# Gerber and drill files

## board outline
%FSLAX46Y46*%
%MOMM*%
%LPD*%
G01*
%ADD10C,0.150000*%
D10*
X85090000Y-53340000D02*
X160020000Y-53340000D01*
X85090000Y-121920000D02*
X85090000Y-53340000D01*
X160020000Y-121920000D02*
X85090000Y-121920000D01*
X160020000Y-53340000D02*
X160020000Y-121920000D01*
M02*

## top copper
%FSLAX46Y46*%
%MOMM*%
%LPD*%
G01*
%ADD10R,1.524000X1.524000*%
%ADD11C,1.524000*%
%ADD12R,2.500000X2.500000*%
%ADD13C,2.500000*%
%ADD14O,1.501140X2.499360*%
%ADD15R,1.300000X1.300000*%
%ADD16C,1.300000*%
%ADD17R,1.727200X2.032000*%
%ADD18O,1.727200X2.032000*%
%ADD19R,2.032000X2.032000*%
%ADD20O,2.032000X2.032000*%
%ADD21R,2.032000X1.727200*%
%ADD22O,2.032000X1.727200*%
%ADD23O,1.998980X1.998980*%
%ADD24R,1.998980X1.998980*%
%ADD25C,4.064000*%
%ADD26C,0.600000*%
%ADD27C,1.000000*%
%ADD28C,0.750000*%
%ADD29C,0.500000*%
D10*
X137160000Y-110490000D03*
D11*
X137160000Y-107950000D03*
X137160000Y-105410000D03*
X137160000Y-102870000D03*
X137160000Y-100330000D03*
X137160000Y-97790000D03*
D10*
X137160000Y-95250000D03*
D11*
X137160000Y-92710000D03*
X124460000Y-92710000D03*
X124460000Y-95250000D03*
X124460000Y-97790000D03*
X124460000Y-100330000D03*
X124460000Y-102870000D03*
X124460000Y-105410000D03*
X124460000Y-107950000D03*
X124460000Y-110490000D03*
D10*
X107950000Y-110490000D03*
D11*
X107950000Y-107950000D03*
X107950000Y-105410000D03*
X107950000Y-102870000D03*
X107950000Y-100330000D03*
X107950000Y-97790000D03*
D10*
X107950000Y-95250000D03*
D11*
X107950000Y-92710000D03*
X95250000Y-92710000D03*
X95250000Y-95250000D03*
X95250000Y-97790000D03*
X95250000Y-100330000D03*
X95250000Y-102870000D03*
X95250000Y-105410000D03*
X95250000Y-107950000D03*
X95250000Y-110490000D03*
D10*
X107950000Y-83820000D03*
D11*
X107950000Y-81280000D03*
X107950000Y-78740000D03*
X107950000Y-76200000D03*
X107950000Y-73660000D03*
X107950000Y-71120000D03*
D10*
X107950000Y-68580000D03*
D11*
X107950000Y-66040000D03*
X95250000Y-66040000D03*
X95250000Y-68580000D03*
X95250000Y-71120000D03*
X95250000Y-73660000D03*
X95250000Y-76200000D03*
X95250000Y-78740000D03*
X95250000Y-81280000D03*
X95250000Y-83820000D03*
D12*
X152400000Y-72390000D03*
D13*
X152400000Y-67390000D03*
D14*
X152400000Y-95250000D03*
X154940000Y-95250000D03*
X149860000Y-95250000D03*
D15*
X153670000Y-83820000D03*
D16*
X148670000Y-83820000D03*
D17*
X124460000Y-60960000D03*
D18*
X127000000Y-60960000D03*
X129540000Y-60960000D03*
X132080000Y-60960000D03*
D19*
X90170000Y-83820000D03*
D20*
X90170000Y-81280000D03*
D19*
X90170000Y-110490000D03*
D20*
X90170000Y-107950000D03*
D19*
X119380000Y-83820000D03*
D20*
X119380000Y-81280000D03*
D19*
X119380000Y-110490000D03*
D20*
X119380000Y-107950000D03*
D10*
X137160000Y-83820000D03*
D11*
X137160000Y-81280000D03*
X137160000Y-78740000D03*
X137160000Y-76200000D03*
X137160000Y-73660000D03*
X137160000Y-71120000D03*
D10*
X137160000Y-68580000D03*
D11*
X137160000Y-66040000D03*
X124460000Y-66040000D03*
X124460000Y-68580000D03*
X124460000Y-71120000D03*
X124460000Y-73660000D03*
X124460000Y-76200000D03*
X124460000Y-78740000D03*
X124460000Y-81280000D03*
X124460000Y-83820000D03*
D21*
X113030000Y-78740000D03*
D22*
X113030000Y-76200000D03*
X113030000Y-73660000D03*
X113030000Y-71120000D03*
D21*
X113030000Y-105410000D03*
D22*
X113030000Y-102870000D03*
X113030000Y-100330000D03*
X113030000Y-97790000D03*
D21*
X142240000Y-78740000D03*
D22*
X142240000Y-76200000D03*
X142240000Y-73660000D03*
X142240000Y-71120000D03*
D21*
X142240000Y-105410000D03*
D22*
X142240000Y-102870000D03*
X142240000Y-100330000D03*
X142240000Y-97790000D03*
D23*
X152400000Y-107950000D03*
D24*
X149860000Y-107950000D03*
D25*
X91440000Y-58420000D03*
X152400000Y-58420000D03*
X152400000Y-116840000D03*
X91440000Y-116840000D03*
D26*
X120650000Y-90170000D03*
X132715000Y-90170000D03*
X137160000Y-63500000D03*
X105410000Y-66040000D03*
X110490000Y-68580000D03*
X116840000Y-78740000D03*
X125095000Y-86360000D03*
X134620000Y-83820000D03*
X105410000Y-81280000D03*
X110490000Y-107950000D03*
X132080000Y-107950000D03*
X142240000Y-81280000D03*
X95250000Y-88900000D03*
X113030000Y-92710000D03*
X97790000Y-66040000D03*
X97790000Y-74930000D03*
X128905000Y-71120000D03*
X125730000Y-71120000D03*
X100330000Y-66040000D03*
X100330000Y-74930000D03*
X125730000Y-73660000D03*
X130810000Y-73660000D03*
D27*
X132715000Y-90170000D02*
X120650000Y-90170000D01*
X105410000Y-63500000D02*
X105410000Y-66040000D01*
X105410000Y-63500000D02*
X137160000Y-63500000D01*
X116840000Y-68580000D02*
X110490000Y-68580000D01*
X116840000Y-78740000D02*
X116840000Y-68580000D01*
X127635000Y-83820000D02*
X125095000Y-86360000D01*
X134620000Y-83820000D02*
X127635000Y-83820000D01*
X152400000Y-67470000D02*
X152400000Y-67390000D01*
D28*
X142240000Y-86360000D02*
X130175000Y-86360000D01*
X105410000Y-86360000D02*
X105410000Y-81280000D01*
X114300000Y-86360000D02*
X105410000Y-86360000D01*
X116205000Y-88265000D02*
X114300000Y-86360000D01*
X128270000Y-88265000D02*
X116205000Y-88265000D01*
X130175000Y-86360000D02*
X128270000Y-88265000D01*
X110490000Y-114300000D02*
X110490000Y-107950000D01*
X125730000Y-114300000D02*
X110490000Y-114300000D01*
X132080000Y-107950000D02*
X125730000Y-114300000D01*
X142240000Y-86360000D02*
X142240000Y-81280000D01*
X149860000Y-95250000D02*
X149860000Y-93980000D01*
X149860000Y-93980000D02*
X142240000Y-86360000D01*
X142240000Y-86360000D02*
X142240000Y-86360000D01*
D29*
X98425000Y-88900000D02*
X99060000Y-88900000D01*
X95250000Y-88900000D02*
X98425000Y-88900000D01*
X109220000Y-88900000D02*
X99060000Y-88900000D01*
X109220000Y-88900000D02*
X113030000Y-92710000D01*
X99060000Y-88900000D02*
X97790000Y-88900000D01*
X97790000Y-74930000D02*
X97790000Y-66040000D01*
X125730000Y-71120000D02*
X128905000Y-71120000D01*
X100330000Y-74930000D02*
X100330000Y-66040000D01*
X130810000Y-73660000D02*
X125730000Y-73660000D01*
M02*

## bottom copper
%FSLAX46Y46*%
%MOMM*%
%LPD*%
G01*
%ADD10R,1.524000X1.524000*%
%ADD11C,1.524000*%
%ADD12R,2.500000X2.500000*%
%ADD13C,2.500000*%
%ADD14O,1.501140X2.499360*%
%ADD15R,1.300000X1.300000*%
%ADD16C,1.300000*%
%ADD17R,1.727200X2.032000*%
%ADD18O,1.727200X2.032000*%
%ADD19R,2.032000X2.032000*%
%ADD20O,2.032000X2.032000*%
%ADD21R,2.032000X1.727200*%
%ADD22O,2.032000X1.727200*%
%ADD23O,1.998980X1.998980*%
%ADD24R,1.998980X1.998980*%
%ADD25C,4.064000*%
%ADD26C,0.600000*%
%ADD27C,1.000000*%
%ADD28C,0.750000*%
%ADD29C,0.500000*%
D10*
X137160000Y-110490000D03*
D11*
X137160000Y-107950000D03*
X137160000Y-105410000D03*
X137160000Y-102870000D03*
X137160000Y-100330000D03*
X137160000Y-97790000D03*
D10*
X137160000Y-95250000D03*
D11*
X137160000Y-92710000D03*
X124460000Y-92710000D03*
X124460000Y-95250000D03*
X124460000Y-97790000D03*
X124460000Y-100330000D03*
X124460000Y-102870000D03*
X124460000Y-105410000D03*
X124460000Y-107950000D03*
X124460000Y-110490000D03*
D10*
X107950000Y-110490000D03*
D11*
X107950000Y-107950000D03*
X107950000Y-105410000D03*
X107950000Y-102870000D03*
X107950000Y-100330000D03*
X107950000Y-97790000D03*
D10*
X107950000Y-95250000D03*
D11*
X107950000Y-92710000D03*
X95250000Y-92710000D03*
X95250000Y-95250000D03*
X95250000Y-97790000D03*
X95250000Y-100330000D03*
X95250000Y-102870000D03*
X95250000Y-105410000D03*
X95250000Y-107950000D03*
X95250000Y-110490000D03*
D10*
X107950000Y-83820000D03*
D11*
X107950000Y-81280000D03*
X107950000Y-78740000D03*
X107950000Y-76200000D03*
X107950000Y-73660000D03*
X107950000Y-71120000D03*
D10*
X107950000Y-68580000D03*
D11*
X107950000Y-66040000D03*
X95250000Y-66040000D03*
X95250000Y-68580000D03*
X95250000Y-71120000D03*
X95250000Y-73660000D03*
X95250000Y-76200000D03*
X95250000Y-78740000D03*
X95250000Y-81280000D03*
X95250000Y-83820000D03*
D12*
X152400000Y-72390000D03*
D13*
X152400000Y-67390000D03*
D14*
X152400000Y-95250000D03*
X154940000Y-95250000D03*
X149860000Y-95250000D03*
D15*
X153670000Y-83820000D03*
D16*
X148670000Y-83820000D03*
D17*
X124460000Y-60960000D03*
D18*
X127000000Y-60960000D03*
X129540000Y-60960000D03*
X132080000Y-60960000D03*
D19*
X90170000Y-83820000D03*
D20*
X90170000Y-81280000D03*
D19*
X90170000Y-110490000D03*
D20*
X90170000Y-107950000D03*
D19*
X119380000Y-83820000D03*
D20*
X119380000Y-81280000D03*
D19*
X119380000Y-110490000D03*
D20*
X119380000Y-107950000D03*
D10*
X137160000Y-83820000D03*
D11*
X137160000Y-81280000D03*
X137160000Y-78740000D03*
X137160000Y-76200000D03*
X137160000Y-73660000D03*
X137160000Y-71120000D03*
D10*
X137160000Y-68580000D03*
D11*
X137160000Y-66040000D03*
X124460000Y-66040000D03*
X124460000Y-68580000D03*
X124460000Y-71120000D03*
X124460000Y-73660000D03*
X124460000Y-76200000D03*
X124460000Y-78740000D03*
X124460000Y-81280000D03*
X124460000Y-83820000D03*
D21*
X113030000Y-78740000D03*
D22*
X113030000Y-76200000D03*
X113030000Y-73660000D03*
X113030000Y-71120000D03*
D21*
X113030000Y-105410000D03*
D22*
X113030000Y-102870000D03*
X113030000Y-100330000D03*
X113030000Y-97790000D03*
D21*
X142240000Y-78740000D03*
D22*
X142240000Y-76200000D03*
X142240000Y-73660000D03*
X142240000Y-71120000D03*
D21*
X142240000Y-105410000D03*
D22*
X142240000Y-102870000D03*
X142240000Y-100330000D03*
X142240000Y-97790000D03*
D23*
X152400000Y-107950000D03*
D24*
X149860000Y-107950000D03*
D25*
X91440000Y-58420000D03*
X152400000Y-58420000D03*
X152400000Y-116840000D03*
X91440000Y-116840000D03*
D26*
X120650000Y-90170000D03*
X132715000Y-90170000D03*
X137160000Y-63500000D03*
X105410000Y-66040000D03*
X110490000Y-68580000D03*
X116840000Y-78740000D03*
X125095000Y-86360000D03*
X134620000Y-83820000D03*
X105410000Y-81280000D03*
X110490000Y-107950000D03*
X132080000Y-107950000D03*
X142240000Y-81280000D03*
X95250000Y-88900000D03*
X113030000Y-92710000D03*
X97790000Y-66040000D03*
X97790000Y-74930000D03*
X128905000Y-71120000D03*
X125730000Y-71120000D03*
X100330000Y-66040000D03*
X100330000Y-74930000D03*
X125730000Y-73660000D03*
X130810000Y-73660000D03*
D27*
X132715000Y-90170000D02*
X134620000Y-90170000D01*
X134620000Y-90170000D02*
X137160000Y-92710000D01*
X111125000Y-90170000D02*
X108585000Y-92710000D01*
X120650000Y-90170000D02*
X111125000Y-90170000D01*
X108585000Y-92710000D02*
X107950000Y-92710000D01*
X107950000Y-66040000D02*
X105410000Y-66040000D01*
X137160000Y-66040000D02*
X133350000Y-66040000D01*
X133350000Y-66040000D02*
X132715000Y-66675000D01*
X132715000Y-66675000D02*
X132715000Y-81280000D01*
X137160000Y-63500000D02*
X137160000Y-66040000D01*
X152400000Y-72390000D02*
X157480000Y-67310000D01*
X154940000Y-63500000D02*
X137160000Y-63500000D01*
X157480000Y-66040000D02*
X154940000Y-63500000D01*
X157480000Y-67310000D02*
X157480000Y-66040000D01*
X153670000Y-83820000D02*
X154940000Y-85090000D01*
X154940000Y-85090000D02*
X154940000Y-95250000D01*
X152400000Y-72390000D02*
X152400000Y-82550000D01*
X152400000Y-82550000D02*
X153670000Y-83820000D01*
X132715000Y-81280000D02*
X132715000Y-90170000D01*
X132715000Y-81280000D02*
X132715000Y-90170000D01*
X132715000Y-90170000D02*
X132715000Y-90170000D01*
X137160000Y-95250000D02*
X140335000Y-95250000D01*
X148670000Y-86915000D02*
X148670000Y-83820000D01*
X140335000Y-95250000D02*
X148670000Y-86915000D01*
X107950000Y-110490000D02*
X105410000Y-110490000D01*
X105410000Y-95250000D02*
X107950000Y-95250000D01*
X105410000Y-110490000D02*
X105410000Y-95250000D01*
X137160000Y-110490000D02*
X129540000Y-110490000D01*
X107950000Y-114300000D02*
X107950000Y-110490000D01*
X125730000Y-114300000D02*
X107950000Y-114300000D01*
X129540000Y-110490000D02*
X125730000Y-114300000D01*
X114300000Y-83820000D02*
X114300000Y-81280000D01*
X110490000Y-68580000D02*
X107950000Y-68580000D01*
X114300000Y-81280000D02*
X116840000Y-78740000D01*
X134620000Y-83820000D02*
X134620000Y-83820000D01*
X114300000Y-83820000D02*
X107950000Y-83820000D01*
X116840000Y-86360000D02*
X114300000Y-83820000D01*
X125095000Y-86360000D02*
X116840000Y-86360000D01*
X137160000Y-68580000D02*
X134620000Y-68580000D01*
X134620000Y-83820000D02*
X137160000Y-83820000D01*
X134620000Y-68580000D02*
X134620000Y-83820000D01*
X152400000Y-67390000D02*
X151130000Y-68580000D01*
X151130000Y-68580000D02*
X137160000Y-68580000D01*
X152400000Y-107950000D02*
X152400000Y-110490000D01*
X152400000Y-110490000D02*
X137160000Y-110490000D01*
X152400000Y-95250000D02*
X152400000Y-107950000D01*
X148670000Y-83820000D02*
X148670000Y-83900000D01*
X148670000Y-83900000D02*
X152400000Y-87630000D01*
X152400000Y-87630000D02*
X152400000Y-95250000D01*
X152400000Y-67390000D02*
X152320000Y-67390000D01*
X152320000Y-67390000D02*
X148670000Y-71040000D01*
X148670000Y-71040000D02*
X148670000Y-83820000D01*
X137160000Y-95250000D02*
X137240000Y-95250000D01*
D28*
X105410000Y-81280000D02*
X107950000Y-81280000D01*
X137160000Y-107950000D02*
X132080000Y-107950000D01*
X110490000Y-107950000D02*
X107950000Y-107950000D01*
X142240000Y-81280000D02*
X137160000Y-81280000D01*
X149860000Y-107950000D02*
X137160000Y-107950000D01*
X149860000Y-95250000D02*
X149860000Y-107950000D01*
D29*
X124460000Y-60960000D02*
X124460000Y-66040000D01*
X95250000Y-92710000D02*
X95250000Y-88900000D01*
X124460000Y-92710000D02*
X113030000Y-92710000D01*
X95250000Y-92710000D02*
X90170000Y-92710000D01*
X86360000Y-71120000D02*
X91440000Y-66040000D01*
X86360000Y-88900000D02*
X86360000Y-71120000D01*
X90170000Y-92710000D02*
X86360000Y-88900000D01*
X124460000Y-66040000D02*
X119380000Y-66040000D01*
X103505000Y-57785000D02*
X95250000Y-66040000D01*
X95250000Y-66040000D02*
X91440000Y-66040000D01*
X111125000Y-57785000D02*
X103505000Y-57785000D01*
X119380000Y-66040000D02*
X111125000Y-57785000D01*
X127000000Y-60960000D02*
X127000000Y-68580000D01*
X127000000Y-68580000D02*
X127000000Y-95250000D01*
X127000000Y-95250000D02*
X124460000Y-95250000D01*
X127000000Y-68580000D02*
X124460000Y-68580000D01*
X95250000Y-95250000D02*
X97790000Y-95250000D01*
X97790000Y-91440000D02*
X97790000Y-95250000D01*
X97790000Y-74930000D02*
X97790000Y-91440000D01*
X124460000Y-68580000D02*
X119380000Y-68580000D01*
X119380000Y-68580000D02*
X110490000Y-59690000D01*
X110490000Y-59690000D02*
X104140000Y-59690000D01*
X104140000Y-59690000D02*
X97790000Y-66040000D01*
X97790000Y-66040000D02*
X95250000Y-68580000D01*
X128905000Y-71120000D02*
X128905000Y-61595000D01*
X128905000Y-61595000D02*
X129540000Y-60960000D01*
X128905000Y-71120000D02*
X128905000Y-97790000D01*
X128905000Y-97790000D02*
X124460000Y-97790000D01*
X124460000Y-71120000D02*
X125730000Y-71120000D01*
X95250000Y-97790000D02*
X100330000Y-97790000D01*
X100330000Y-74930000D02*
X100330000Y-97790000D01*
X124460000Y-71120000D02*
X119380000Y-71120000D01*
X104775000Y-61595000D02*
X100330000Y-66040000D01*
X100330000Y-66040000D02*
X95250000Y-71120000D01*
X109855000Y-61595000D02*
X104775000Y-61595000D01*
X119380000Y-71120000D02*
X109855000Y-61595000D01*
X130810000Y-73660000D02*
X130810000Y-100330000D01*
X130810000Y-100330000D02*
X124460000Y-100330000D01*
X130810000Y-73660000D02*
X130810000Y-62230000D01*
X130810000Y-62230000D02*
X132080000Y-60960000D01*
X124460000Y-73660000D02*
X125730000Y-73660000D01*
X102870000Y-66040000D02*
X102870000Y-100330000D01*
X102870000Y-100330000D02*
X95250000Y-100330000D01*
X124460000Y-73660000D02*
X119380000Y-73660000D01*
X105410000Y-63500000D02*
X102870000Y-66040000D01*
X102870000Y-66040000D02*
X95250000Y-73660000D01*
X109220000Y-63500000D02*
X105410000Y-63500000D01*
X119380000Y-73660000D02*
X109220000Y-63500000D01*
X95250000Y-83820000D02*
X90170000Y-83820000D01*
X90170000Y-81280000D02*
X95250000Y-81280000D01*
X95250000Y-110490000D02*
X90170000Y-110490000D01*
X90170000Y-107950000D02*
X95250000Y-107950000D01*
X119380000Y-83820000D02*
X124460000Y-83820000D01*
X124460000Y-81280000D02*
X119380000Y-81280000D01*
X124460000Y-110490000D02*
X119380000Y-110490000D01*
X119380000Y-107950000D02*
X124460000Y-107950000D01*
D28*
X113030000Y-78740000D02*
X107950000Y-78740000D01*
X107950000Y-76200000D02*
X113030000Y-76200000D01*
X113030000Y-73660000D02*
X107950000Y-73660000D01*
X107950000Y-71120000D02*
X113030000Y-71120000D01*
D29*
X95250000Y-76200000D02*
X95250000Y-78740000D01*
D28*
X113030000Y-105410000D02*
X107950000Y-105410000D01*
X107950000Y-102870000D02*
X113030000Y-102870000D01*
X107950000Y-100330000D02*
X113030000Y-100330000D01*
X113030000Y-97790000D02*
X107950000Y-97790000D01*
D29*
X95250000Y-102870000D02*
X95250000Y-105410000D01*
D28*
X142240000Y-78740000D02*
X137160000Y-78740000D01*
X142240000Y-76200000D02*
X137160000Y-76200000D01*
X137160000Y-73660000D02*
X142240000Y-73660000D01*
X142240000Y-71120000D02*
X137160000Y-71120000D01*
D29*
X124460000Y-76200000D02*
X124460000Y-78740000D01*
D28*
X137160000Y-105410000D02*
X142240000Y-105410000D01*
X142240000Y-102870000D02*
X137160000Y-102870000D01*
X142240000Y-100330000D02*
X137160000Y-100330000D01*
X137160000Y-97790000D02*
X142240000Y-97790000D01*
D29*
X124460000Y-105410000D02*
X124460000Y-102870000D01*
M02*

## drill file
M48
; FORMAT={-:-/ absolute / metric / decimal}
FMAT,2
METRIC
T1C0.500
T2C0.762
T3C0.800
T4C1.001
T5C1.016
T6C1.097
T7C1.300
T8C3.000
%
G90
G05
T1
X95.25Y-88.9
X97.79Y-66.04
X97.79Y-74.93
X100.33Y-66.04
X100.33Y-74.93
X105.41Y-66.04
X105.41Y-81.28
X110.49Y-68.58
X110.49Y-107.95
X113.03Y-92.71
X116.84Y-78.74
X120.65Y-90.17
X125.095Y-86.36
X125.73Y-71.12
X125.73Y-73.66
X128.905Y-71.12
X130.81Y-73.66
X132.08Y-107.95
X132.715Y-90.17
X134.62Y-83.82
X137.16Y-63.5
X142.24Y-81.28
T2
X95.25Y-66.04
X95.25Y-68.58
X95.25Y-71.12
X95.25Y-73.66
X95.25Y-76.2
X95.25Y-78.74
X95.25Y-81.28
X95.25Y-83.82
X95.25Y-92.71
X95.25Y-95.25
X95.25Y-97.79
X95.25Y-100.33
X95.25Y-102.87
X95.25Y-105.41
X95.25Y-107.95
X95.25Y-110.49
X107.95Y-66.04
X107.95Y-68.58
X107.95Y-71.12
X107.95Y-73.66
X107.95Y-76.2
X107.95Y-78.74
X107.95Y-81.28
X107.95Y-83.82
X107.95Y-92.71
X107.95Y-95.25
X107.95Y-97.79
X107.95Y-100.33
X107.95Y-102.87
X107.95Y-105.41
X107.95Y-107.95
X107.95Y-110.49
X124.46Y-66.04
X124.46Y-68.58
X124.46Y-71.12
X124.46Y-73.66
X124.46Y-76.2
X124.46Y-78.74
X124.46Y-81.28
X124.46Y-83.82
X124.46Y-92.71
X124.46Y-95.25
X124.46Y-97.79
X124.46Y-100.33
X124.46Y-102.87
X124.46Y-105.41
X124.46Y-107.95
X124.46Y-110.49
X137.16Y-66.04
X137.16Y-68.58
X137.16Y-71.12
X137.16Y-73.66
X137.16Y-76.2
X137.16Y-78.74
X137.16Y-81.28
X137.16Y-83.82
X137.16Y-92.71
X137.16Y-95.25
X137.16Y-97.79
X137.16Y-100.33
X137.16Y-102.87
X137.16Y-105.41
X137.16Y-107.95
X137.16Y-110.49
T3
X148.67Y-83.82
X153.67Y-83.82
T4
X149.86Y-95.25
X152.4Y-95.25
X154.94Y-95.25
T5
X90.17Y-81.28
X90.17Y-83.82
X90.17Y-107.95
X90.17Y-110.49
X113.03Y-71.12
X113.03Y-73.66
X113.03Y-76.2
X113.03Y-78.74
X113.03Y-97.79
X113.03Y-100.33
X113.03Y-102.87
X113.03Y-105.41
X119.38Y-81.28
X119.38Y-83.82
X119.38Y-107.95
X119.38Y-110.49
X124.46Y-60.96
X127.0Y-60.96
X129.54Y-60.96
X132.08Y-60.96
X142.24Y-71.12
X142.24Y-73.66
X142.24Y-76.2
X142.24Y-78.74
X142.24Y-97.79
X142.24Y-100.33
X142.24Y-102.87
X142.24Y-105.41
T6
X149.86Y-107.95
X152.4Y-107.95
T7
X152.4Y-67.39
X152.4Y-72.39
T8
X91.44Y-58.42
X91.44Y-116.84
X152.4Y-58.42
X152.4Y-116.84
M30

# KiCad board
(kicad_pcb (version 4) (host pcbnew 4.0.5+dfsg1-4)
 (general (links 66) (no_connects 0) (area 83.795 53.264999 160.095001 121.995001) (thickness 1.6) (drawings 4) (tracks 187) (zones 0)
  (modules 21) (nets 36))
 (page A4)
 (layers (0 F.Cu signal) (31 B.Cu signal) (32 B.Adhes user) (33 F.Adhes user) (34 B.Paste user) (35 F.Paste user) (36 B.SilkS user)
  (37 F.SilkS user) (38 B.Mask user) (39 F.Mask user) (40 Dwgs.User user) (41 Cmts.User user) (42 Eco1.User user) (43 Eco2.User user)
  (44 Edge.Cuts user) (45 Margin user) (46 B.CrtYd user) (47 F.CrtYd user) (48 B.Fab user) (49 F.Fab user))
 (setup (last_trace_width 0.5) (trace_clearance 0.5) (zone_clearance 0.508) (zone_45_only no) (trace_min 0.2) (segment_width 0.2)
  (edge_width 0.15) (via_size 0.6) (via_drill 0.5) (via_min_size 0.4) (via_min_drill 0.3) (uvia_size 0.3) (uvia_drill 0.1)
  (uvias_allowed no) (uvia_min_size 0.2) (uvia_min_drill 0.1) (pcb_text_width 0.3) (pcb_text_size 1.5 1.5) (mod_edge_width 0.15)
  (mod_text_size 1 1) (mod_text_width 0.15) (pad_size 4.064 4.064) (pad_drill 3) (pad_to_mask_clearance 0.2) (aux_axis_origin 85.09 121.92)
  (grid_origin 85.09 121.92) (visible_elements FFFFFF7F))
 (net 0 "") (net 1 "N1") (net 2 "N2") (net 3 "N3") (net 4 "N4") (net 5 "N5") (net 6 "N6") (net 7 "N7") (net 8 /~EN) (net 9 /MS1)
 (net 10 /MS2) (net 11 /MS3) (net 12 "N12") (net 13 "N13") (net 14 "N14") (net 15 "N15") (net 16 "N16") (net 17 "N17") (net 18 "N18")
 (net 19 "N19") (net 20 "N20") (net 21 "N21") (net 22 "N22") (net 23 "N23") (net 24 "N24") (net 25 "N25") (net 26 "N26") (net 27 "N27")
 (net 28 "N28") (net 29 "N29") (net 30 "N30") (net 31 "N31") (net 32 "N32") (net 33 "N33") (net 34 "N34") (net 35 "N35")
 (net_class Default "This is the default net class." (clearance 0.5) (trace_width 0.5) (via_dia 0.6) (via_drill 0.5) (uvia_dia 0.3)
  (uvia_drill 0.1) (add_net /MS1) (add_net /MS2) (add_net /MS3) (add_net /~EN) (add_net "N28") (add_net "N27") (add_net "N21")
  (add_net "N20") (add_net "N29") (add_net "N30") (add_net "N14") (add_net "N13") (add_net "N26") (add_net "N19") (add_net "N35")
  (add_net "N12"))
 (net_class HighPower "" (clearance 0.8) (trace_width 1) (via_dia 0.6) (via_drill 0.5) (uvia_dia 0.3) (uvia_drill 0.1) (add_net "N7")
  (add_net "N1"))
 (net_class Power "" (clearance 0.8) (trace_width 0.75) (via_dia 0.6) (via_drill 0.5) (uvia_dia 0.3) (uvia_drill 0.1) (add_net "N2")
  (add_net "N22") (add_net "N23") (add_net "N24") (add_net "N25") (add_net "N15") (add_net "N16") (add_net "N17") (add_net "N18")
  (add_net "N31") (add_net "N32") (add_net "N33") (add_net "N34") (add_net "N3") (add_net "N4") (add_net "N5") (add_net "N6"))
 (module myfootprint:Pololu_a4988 (layer F.Cu) (at 130.81 101.6)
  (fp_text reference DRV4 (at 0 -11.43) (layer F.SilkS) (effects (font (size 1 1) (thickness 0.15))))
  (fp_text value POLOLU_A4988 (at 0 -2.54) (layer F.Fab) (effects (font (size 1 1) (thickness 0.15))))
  (pad 1 thru_hole rect (at 6.35 8.89) (size 1.524 1.524) (drill 0.762) (layers *.Cu *.Mask) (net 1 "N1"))
  (pad 2 thru_hole circle (at 6.35 6.35) (size 1.524 1.524) (drill 0.762) (layers *.Cu *.Mask) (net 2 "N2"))
  (pad 3 thru_hole circle (at 6.35 3.81) (size 1.524 1.524) (drill 0.762) (layers *.Cu *.Mask) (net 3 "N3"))
  (pad 4 thru_hole circle (at 6.35 1.27) (size 1.524 1.524) (drill 0.762) (layers *.Cu *.Mask) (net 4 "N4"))
  (pad 5 thru_hole circle (at 6.35 -1.27) (size 1.524 1.524) (drill 0.762) (layers *.Cu *.Mask) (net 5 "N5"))
  (pad 6 thru_hole circle (at 6.35 -3.81) (size 1.524 1.524) (drill 0.762) (layers *.Cu *.Mask) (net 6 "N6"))
  (pad 7 thru_hole rect (at 6.35 -6.35) (size 1.524 1.524) (drill 0.762) (layers *.Cu *.Mask) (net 1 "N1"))
  (pad 8 thru_hole circle (at 6.35 -8.89) (size 1.524 1.524) (drill 0.762) (layers *.Cu *.Mask) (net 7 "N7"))
  (pad 9 thru_hole circle (at -6.35 -8.89) (size 1.524 1.524) (drill 0.762) (layers *.Cu *.Mask) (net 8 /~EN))
  (pad 10 thru_hole circle (at -6.35 -6.35) (size 1.524 1.524) (drill 0.762) (layers *.Cu *.Mask) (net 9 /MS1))
  (pad 11 thru_hole circle (at -6.35 -3.81) (size 1.524 1.524) (drill 0.762) (layers *.Cu *.Mask) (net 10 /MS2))
  (pad 12 thru_hole circle (at -6.35 -1.27) (size 1.524 1.524) (drill 0.762) (layers *.Cu *.Mask) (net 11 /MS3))
  (pad 13 thru_hole circle (at -6.35 1.27) (size 1.524 1.524) (drill 0.762) (layers *.Cu *.Mask) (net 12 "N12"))
  (pad 14 thru_hole circle (at -6.35 3.81) (size 1.524 1.524) (drill 0.762) (layers *.Cu *.Mask) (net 12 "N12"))
  (pad 15 thru_hole circle (at -6.35 6.35) (size 1.524 1.524) (drill 0.762) (layers *.Cu *.Mask) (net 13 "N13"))
  (pad 16 thru_hole circle (at -6.35 8.89) (size 1.524 1.524) (drill 0.762) (layers *.Cu *.Mask) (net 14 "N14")))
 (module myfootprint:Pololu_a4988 (layer F.Cu) (at 101.6 101.6)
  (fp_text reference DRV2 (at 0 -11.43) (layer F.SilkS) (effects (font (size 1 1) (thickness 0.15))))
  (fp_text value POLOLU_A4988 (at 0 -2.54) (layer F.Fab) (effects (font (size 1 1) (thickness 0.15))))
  (pad 1 thru_hole rect (at 6.35 8.89) (size 1.524 1.524) (drill 0.762) (layers *.Cu *.Mask) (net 1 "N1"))
  (pad 2 thru_hole circle (at 6.35 6.35) (size 1.524 1.524) (drill 0.762) (layers *.Cu *.Mask) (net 2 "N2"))
  (pad 3 thru_hole circle (at 6.35 3.81) (size 1.524 1.524) (drill 0.762) (layers *.Cu *.Mask) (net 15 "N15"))
  (pad 4 thru_hole circle (at 6.35 1.27) (size 1.524 1.524) (drill 0.762) (layers *.Cu *.Mask) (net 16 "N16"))
  (pad 5 thru_hole circle (at 6.35 -1.27) (size 1.524 1.524) (drill 0.762) (layers *.Cu *.Mask) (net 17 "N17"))
  (pad 6 thru_hole circle (at 6.35 -3.81) (size 1.524 1.524) (drill 0.762) (layers *.Cu *.Mask) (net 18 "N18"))
  (pad 7 thru_hole rect (at 6.35 -6.35) (size 1.524 1.524) (drill 0.762) (layers *.Cu *.Mask) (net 1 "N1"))
  (pad 8 thru_hole circle (at 6.35 -8.89) (size 1.524 1.524) (drill 0.762) (layers *.Cu *.Mask) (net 7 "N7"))
  (pad 9 thru_hole circle (at -6.35 -8.89) (size 1.524 1.524) (drill 0.762) (layers *.Cu *.Mask) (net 8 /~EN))
  (pad 10 thru_hole circle (at -6.35 -6.35) (size 1.524 1.524) (drill 0.762) (layers *.Cu *.Mask) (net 9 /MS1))
  (pad 11 thru_hole circle (at -6.35 -3.81) (size 1.524 1.524) (drill 0.762) (layers *.Cu *.Mask) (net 10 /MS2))
  (pad 12 thru_hole circle (at -6.35 -1.27) (size 1.524 1.524) (drill 0.762) (layers *.Cu *.Mask) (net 11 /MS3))
  (pad 13 thru_hole circle (at -6.35 1.27) (size 1.524 1.524) (drill 0.762) (layers *.Cu *.Mask) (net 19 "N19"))
  (pad 14 thru_hole circle (at -6.35 3.81) (size 1.524 1.524) (drill 0.762) (layers *.Cu *.Mask) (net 19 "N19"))
  (pad 15 thru_hole circle (at -6.35 6.35) (size 1.524 1.524) (drill 0.762) (layers *.Cu *.Mask) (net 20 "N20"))
  (pad 16 thru_hole circle (at -6.35 8.89) (size 1.524 1.524) (drill 0.762) (layers *.Cu *.Mask) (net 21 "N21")))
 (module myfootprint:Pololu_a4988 (layer F.Cu) (at 101.6 74.93)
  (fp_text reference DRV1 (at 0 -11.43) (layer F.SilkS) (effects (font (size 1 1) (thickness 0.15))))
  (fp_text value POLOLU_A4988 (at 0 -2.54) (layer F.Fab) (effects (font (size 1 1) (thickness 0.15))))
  (pad 1 thru_hole rect (at 6.35 8.89) (size 1.524 1.524) (drill 0.762) (layers *.Cu *.Mask) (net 1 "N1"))
  (pad 2 thru_hole circle (at 6.35 6.35) (size 1.524 1.524) (drill 0.762) (layers *.Cu *.Mask) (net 2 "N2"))
  (pad 3 thru_hole circle (at 6.35 3.81) (size 1.524 1.524) (drill 0.762) (layers *.Cu *.Mask) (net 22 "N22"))
  (pad 4 thru_hole circle (at 6.35 1.27) (size 1.524 1.524) (drill 0.762) (layers *.Cu *.Mask) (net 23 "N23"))
  (pad 5 thru_hole circle (at 6.35 -1.27) (size 1.524 1.524) (drill 0.762) (layers *.Cu *.Mask) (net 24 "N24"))
  (pad 6 thru_hole circle (at 6.35 -3.81) (size 1.524 1.524) (drill 0.762) (layers *.Cu *.Mask) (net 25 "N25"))
  (pad 7 thru_hole rect (at 6.35 -6.35) (size 1.524 1.524) (drill 0.762) (layers *.Cu *.Mask) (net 1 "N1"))
  (pad 8 thru_hole circle (at 6.35 -8.89) (size 1.524 1.524) (drill 0.762) (layers *.Cu *.Mask) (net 7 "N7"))
  (pad 9 thru_hole circle (at -6.35 -8.89) (size 1.524 1.524) (drill 0.762) (layers *.Cu *.Mask) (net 8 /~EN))
  (pad 10 thru_hole circle (at -6.35 -6.35) (size 1.524 1.524) (drill 0.762) (layers *.Cu *.Mask) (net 9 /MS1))
  (pad 11 thru_hole circle (at -6.35 -3.81) (size 1.524 1.524) (drill 0.762) (layers *.Cu *.Mask) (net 10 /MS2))
  (pad 12 thru_hole circle (at -6.35 -1.27) (size 1.524 1.524) (drill 0.762) (layers *.Cu *.Mask) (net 11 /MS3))
  (pad 13 thru_hole circle (at -6.35 1.27) (size 1.524 1.524) (drill 0.762) (layers *.Cu *.Mask) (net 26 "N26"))
  (pad 14 thru_hole circle (at -6.35 3.81) (size 1.524 1.524) (drill 0.762) (layers *.Cu *.Mask) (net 26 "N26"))
  (pad 15 thru_hole circle (at -6.35 6.35) (size 1.524 1.524) (drill 0.762) (layers *.Cu *.Mask) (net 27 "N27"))
  (pad 16 thru_hole circle (at -6.35 8.89) (size 1.524 1.524) (drill 0.762) (layers *.Cu *.Mask) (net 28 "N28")))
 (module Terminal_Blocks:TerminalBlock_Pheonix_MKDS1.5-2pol (layer F.Cu) (at 152.4 72.39 90)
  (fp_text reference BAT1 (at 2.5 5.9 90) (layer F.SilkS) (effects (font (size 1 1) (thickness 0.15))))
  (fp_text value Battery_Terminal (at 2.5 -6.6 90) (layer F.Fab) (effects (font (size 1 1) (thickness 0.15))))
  (pad 1 thru_hole rect (at 0 0 90) (size 2.5 2.5) (drill 1.3) (layers *.Cu *.Mask) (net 7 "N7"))
  (pad 2 thru_hole circle (at 5 0 90) (size 2.5 2.5) (drill 1.3) (layers *.Cu *.Mask) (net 1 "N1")))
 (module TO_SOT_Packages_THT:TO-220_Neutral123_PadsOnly (layer F.Cu) (at 152.4 95.25 180)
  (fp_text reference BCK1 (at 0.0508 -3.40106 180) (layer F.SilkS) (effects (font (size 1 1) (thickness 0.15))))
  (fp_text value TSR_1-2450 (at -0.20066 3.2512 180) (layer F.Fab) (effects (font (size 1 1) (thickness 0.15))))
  (pad 2 thru_hole oval (at 0 0 270) (size 2.49936 1.50114) (drill 1.00076) (layers *.Cu *.Mask) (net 1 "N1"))
  (pad 1 thru_hole oval (at -2.54 0 270) (size 2.49936 1.50114) (drill 1.00076) (layers *.Cu *.Mask) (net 7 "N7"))
  (pad 3 thru_hole oval (at 2.54 0 270) (size 2.49936 1.50114) (drill 1.00076) (layers *.Cu *.Mask) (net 2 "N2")))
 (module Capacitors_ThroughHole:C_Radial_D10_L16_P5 (layer F.Cu) (at 153.67 83.82 180)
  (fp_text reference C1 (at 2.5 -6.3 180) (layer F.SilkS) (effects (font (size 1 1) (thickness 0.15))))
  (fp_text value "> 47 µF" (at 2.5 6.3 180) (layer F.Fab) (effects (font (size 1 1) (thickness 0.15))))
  (pad 1 thru_hole rect (at 0 0 180) (size 1.3 1.3) (drill 0.8) (layers *.Cu *.Mask) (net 7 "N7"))
  (pad 2 thru_hole circle (at 5 0 180) (size 1.3 1.3) (drill 0.8) (layers *.Cu *.Mask) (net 1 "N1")))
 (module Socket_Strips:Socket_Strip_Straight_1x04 (layer F.Cu) (at 124.46 60.96)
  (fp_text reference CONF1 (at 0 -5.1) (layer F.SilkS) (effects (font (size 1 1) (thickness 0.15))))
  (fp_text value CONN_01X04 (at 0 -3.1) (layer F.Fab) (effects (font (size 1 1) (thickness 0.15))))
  (pad 1 thru_hole rect (at 0 0) (size 1.7272 2.032) (drill 1.016) (layers *.Cu *.Mask) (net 8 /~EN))
  (pad 2 thru_hole oval (at 2.54 0) (size 1.7272 2.032) (drill 1.016) (layers *.Cu *.Mask) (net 9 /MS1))
  (pad 3 thru_hole oval (at 5.08 0) (size 1.7272 2.032) (drill 1.016) (layers *.Cu *.Mask) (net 10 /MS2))
  (pad 4 thru_hole oval (at 7.62 0) (size 1.7272 2.032) (drill 1.016) (layers *.Cu *.Mask) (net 11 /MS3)))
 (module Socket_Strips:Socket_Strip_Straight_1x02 (layer F.Cu) (at 90.17 83.82 90)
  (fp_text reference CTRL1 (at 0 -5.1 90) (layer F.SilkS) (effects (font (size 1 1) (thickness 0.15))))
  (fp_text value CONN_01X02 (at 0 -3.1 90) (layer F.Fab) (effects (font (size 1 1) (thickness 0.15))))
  (pad 1 thru_hole rect (at 0 0 90) (size 2.032 2.032) (drill 1.016) (layers *.Cu *.Mask) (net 28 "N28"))
  (pad 2 thru_hole oval (at 2.54 0 90) (size 2.032 2.032) (drill 1.016) (layers *.Cu *.Mask) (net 27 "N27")))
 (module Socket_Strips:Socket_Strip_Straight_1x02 (layer F.Cu) (at 90.17 110.49 90)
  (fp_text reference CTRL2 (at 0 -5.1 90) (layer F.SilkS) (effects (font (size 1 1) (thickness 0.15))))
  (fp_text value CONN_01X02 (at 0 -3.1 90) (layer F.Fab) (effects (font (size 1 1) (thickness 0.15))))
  (pad 1 thru_hole rect (at 0 0 90) (size 2.032 2.032) (drill 1.016) (layers *.Cu *.Mask) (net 21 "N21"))
  (pad 2 thru_hole oval (at 2.54 0 90) (size 2.032 2.032) (drill 1.016) (layers *.Cu *.Mask) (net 20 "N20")))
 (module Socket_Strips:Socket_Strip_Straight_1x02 (layer F.Cu) (at 119.38 83.82 90)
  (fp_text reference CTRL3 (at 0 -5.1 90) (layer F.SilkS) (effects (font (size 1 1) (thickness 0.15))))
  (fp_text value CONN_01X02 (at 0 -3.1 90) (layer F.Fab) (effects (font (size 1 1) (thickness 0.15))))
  (pad 1 thru_hole rect (at 0 0 90) (size 2.032 2.032) (drill 1.016) (layers *.Cu *.Mask) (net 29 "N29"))
  (pad 2 thru_hole oval (at 2.54 0 90) (size 2.032 2.032) (drill 1.016) (layers *.Cu *.Mask) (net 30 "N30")))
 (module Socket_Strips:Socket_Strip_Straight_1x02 (layer F.Cu) (at 119.38 110.49 90)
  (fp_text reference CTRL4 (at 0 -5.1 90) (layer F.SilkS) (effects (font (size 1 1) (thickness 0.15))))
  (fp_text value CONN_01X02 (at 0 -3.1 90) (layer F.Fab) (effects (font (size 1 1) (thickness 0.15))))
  (pad 1 thru_hole rect (at 0 0 90) (size 2.032 2.032) (drill 1.016) (layers *.Cu *.Mask) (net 14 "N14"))
  (pad 2 thru_hole oval (at 2.54 0 90) (size 2.032 2.032) (drill 1.016) (layers *.Cu *.Mask) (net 13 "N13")))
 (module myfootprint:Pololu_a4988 (layer F.Cu) (at 130.81 74.93)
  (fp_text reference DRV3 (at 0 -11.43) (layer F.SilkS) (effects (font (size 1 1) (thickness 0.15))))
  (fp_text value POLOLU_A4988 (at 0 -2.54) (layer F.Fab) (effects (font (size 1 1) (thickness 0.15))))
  (pad 1 thru_hole rect (at 6.35 8.89) (size 1.524 1.524) (drill 0.762) (layers *.Cu *.Mask) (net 1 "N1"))
  (pad 2 thru_hole circle (at 6.35 6.35) (size 1.524 1.524) (drill 0.762) (layers *.Cu *.Mask) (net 2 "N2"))
  (pad 3 thru_hole circle (at 6.35 3.81) (size 1.524 1.524) (drill 0.762) (layers *.Cu *.Mask) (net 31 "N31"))
  (pad 4 thru_hole circle (at 6.35 1.27) (size 1.524 1.524) (drill 0.762) (layers *.Cu *.Mask) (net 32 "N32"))
  (pad 5 thru_hole circle (at 6.35 -1.27) (size 1.524 1.524) (drill 0.762) (layers *.Cu *.Mask) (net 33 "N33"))
  (pad 6 thru_hole circle (at 6.35 -3.81) (size 1.524 1.524) (drill 0.762) (layers *.Cu *.Mask) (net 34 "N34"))
  (pad 7 thru_hole rect (at 6.35 -6.35) (size 1.524 1.524) (drill 0.762) (layers *.Cu *.Mask) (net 1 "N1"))
  (pad 8 thru_hole circle (at 6.35 -8.89) (size 1.524 1.524) (drill 0.762) (layers *.Cu *.Mask) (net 7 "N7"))
  (pad 9 thru_hole circle (at -6.35 -8.89) (size 1.524 1.524) (drill 0.762) (layers *.Cu *.Mask) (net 8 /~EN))
  (pad 10 thru_hole circle (at -6.35 -6.35) (size 1.524 1.524) (drill 0.762) (layers *.Cu *.Mask) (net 9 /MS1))
  (pad 11 thru_hole circle (at -6.35 -3.81) (size 1.524 1.524) (drill 0.762) (layers *.Cu *.Mask) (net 10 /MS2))
  (pad 12 thru_hole circle (at -6.35 -1.27) (size 1.524 1.524) (drill 0.762) (layers *.Cu *.Mask) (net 11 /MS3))
  (pad 13 thru_hole circle (at -6.35 1.27) (size 1.524 1.524) (drill 0.762) (layers *.Cu *.Mask) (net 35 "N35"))
  (pad 14 thru_hole circle (at -6.35 3.81) (size 1.524 1.524) (drill 0.762) (layers *.Cu *.Mask) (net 35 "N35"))
  (pad 15 thru_hole circle (at -6.35 6.35) (size 1.524 1.524) (drill 0.762) (layers *.Cu *.Mask) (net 30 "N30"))
  (pad 16 thru_hole circle (at -6.35 8.89) (size 1.524 1.524) (drill 0.762) (layers *.Cu *.Mask) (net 29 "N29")))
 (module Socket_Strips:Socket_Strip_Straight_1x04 (layer F.Cu) (at 113.03 78.74 90)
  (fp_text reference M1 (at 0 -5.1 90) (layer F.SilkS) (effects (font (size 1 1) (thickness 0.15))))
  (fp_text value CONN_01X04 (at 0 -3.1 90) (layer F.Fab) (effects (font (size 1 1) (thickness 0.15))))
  (pad 1 thru_hole rect (at 0 0 90) (size 1.7272 2.032) (drill 1.016) (layers *.Cu *.Mask) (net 22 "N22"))
  (pad 2 thru_hole oval (at 2.54 0 90) (size 1.7272 2.032) (drill 1.016) (layers *.Cu *.Mask) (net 23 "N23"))
  (pad 3 thru_hole oval (at 5.08 0 90) (size 1.7272 2.032) (drill 1.016) (layers *.Cu *.Mask) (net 24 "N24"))
  (pad 4 thru_hole oval (at 7.62 0 90) (size 1.7272 2.032) (drill 1.016) (layers *.Cu *.Mask) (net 25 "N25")))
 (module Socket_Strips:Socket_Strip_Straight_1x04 (layer F.Cu) (at 113.03 105.41 90)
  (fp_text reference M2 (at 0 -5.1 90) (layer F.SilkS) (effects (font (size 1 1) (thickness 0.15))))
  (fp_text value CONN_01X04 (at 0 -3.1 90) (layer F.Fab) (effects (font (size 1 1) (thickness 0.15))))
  (pad 1 thru_hole rect (at 0 0 90) (size 1.7272 2.032) (drill 1.016) (layers *.Cu *.Mask) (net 15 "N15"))
  (pad 2 thru_hole oval (at 2.54 0 90) (size 1.7272 2.032) (drill 1.016) (layers *.Cu *.Mask) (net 16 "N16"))
  (pad 3 thru_hole oval (at 5.08 0 90) (size 1.7272 2.032) (drill 1.016) (layers *.Cu *.Mask) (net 17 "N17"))
  (pad 4 thru_hole oval (at 7.62 0 90) (size 1.7272 2.032) (drill 1.016) (layers *.Cu *.Mask) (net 18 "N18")))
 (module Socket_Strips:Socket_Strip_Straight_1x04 (layer F.Cu) (at 142.24 78.74 90)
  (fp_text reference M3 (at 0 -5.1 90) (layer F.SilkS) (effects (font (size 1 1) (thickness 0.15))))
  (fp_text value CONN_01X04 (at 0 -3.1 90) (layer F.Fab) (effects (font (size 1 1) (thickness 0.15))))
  (pad 1 thru_hole rect (at 0 0 90) (size 1.7272 2.032) (drill 1.016) (layers *.Cu *.Mask) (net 31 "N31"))
  (pad 2 thru_hole oval (at 2.54 0 90) (size 1.7272 2.032) (drill 1.016) (layers *.Cu *.Mask) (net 32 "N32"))
  (pad 3 thru_hole oval (at 5.08 0 90) (size 1.7272 2.032) (drill 1.016) (layers *.Cu *.Mask) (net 33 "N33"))
  (pad 4 thru_hole oval (at 7.62 0 90) (size 1.7272 2.032) (drill 1.016) (layers *.Cu *.Mask) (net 34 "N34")))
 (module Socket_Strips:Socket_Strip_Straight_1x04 (layer F.Cu) (at 142.24 105.41 90)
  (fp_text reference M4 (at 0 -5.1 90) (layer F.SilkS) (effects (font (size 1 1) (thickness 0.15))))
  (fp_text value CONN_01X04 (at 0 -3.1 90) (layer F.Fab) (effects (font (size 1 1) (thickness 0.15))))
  (pad 1 thru_hole rect (at 0 0 90) (size 1.7272 2.032) (drill 1.016) (layers *.Cu *.Mask) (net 3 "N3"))
  (pad 2 thru_hole oval (at 2.54 0 90) (size 1.7272 2.032) (drill 1.016) (layers *.Cu *.Mask) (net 4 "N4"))
  (pad 3 thru_hole oval (at 5.08 0 90) (size 1.7272 2.032) (drill 1.016) (layers *.Cu *.Mask) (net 5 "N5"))
  (pad 4 thru_hole oval (at 7.62 0 90) (size 1.7272 2.032) (drill 1.016) (layers *.Cu *.Mask) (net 6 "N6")))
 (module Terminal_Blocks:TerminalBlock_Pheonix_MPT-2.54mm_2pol (layer F.Cu) (at 149.86 107.95)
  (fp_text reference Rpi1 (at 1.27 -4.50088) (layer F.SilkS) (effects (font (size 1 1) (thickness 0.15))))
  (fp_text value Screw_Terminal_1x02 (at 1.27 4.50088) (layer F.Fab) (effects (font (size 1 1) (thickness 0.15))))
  (pad 2 thru_hole oval (at 2.54 0) (size 1.99898 1.99898) (drill 1.09728) (layers *.Cu *.Mask) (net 1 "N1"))
  (pad 1 thru_hole rect (at 0 0) (size 1.99898 1.99898) (drill 1.09728) (layers *.Cu *.Mask) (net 2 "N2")))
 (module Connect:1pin (layer F.Cu) (at 91.44 58.42)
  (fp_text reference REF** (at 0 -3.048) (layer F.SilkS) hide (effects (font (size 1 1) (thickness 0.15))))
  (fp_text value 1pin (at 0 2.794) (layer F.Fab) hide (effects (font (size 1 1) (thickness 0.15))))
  (pad 1 thru_hole circle (at 0 0) (size 4.064 4.064) (drill 3) (layers *.Cu *.Mask)))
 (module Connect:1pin (layer F.Cu) (at 152.4 58.42)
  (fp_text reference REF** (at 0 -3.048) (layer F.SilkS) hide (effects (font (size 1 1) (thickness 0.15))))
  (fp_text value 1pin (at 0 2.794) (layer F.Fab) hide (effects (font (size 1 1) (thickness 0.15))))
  (pad 1 thru_hole circle (at 0 0) (size 4.064 4.064) (drill 3) (layers *.Cu *.Mask)))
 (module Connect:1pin (layer F.Cu) (at 152.4 116.84)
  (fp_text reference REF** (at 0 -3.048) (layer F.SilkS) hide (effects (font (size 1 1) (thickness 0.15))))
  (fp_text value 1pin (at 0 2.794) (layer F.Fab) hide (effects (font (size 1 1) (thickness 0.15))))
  (pad 1 thru_hole circle (at 0 0) (size 4.064 4.064) (drill 3) (layers *.Cu *.Mask)))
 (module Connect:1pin (layer F.Cu) (at 91.44 116.84)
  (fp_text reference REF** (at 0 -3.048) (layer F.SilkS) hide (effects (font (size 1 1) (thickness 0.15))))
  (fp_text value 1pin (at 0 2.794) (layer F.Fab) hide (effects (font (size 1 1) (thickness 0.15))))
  (pad 1 thru_hole circle (at 0 0) (size 4.064 4.064) (drill 3) (layers *.Cu *.Mask)))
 (gr_line (start 85.09 53.34) (end 160.02 53.34) (angle 90) (layer Edge.Cuts) (width 0.15))
 (gr_line (start 85.09 121.92) (end 85.09 53.34) (angle 90) (layer Edge.Cuts) (width 0.15))
 (gr_line (start 160.02 121.92) (end 85.09 121.92) (angle 90) (layer Edge.Cuts) (width 0.15))
 (gr_line (start 160.02 53.34) (end 160.02 121.92) (angle 90) (layer Edge.Cuts) (width 0.15))
 (segment (start 132.715 90.17) (end 134.62 90.17) (width 1) (layer B.Cu) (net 7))
 (segment (start 134.62 90.17) (end 137.16 92.71) (width 1) (layer B.Cu) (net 7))
 (segment (start 132.715 90.17) (end 120.65 90.17) (width 1) (layer F.Cu) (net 7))
 (segment (start 111.125 90.17) (end 108.585 92.71) (width 1) (layer B.Cu) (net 7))
 (segment (start 120.65 90.17) (end 111.125 90.17) (width 1) (layer B.Cu) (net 7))
 (via (at 120.65 90.17) (size 0.6) (drill 0.5) (layers F.Cu B.Cu) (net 7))
 (segment (start 108.585 92.71) (end 107.95 92.71) (width 1) (layer B.Cu) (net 7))
 (via (at 132.715 90.17) (size 0.6) (drill 0.5) (layers F.Cu B.Cu) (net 7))
 (via (at 137.16 63.5) (size 0.6) (drill 0.5) (layers F.Cu B.Cu) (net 7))
 (segment (start 107.95 66.04) (end 105.41 66.04) (width 1) (layer B.Cu) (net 7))
 (via (at 105.41 66.04) (size 0.6) (drill 0.5) (layers F.Cu B.Cu) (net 7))
 (segment (start 105.41 63.5) (end 105.41 66.04) (width 1) (layer F.Cu) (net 7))
 (segment (start 105.41 63.5) (end 137.16 63.5) (width 1) (layer F.Cu) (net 7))
 (segment (start 137.16 66.04) (end 133.35 66.04) (width 1) (layer B.Cu) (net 7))
 (segment (start 133.35 66.04) (end 132.715 66.675) (width 1) (layer B.Cu) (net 7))
 (segment (start 132.715 66.675) (end 132.715 81.28) (width 1) (layer B.Cu) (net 7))
 (segment (start 137.16 63.5) (end 137.16 66.04) (width 1) (layer B.Cu) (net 7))
 (segment (start 152.4 72.39) (end 157.48 67.31) (width 1) (layer B.Cu) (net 7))
 (segment (start 154.94 63.5) (end 137.16 63.5) (width 1) (layer B.Cu) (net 7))
 (segment (start 157.48 66.04) (end 154.94 63.5) (width 1) (layer B.Cu) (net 7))
 (segment (start 157.48 67.31) (end 157.48 66.04) (width 1) (layer B.Cu) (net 7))
 (segment (start 153.67 83.82) (end 154.94 85.09) (width 1) (layer B.Cu) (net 7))
 (segment (start 154.94 85.09) (end 154.94 95.25) (width 1) (layer B.Cu) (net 7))
 (segment (start 152.4 72.39) (end 152.4 82.55) (width 1) (layer B.Cu) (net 7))
 (segment (start 152.4 82.55) (end 153.67 83.82) (width 1) (layer B.Cu) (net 7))
 (segment (start 132.715 81.28) (end 132.715 90.17) (width 1) (layer B.Cu) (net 7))
 (segment (start 132.715 81.28) (end 132.715 90.17) (width 1) (layer B.Cu) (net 7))
 (segment (start 132.715 90.17) (end 132.715 90.17) (width 1) (layer B.Cu) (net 7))
 (segment (start 137.16 95.25) (end 140.335 95.25) (width 1) (layer B.Cu) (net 1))
 (segment (start 148.67 86.915) (end 148.67 83.82) (width 1) (layer B.Cu) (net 1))
 (segment (start 140.335 95.25) (end 148.67 86.915) (width 1) (layer B.Cu) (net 1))
 (segment (start 107.95 110.49) (end 105.41 110.49) (width 1) (layer B.Cu) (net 1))
 (segment (start 105.41 95.25) (end 107.95 95.25) (width 1) (layer B.Cu) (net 1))
 (segment (start 105.41 110.49) (end 105.41 95.25) (width 1) (layer B.Cu) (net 1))
 (segment (start 137.16 110.49) (end 129.54 110.49) (width 1) (layer B.Cu) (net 1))
 (segment (start 107.95 114.3) (end 107.95 110.49) (width 1) (layer B.Cu) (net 1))
 (segment (start 125.73 114.3) (end 107.95 114.3) (width 1) (layer B.Cu) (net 1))
 (segment (start 129.54 110.49) (end 125.73 114.3) (width 1) (layer B.Cu) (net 1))
 (segment (start 114.3 83.82) (end 114.3 81.28) (width 1) (layer B.Cu) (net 1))
 (segment (start 110.49 68.58) (end 107.95 68.58) (width 1) (layer B.Cu) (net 1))
 (via (at 110.49 68.58) (size 0.6) (drill 0.5) (layers F.Cu B.Cu) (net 1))
 (segment (start 116.84 68.58) (end 110.49 68.58) (width 1) (layer F.Cu) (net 1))
 (segment (start 116.84 78.74) (end 116.84 68.58) (width 1) (layer F.Cu) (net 1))
 (via (at 116.84 78.74) (size 0.6) (drill 0.5) (layers F.Cu B.Cu) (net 1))
 (segment (start 114.3 81.28) (end 116.84 78.74) (width 1) (layer B.Cu) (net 1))
 (segment (start 134.62 83.82) (end 134.62 83.82) (width 1) (layer B.Cu) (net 1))
 (segment (start 114.3 83.82) (end 107.95 83.82) (width 1) (layer B.Cu) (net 1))
 (segment (start 116.84 86.36) (end 114.3 83.82) (width 1) (layer B.Cu) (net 1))
 (segment (start 125.095 86.36) (end 116.84 86.36) (width 1) (layer B.Cu) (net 1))
 (via (at 125.095 86.36) (size 0.6) (drill 0.5) (layers F.Cu B.Cu) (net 1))
 (segment (start 127.635 83.82) (end 125.095 86.36) (width 1) (layer F.Cu) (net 1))
 (segment (start 134.62 83.82) (end 127.635 83.82) (width 1) (layer F.Cu) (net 1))
 (via (at 134.62 83.82) (size 0.6) (drill 0.5) (layers F.Cu B.Cu) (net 1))
 (segment (start 137.16 68.58) (end 134.62 68.58) (width 1) (layer B.Cu) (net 1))
 (segment (start 134.62 83.82) (end 137.16 83.82) (width 1) (layer B.Cu) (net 1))
 (segment (start 134.62 68.58) (end 134.62 83.82) (width 1) (layer B.Cu) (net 1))
 (segment (start 152.4 67.39) (end 151.13 68.58) (width 1) (layer B.Cu) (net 1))
 (segment (start 151.13 68.58) (end 137.16 68.58) (width 1) (layer B.Cu) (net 1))
 (segment (start 152.4 107.95) (end 152.4 110.49) (width 1) (layer B.Cu) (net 1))
 (segment (start 152.4 110.49) (end 137.16 110.49) (width 1) (layer B.Cu) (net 1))
 (segment (start 152.4 95.25) (end 152.4 107.95) (width 1) (layer B.Cu) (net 1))
 (segment (start 148.67 83.82) (end 148.67 83.9) (width 1) (layer B.Cu) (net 1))
 (segment (start 148.67 83.9) (end 152.4 87.63) (width 1) (layer B.Cu) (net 1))
 (segment (start 152.4 87.63) (end 152.4 95.25) (width 1) (layer B.Cu) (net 1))
 (segment (start 152.4 67.39) (end 152.32 67.39) (width 1) (layer B.Cu) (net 1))
 (segment (start 152.32 67.39) (end 148.67 71.04) (width 1) (layer B.Cu) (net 1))
 (segment (start 148.67 71.04) (end 148.67 83.82) (width 1) (layer B.Cu) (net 1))
 (segment (start 137.16 95.25) (end 137.24 95.25) (width 1) (layer B.Cu) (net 1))
 (segment (start 152.4 67.47) (end 152.4 67.39) (width 1) (layer F.Cu) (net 1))
 (segment (start 142.24 86.36) (end 130.175 86.36) (width 0.75) (layer F.Cu) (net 2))
 (segment (start 105.41 81.28) (end 107.95 81.28) (width 0.75) (layer B.Cu) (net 2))
 (via (at 105.41 81.28) (size 0.6) (drill 0.5) (layers F.Cu B.Cu) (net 2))
 (segment (start 105.41 86.36) (end 105.41 81.28) (width 0.75) (layer F.Cu) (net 2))
 (segment (start 114.3 86.36) (end 105.41 86.36) (width 0.75) (layer F.Cu) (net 2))
 (segment (start 116.205 88.265) (end 114.3 86.36) (width 0.75) (layer F.Cu) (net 2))
 (segment (start 128.27 88.265) (end 116.205 88.265) (width 0.75) (layer F.Cu) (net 2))
 (segment (start 130.175 86.36) (end 128.27 88.265) (width 0.75) (layer F.Cu) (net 2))
 (segment (start 137.16 107.95) (end 132.08 107.95) (width 0.75) (layer B.Cu) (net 2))
 (segment (start 110.49 107.95) (end 107.95 107.95) (width 0.75) (layer B.Cu) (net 2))
 (via (at 110.49 107.95) (size 0.6) (drill 0.5) (layers F.Cu B.Cu) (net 2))
 (segment (start 110.49 114.3) (end 110.49 107.95) (width 0.75) (layer F.Cu) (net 2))
 (segment (start 125.73 114.3) (end 110.49 114.3) (width 0.75) (layer F.Cu) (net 2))
 (segment (start 132.08 107.95) (end 125.73 114.3) (width 0.75) (layer F.Cu) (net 2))
 (via (at 132.08 107.95) (size 0.6) (drill 0.5) (layers F.Cu B.Cu) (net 2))
 (segment (start 142.24 86.36) (end 142.24 81.28) (width 0.75) (layer F.Cu) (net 2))
 (segment (start 142.24 81.28) (end 137.16 81.28) (width 0.75) (layer B.Cu) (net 2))
 (via (at 142.24 81.28) (size 0.6) (drill 0.5) (layers F.Cu B.Cu) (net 2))
 (segment (start 149.86 95.25) (end 149.86 93.98) (width 0.75) (layer F.Cu) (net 2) (status 400000))
 (segment (start 149.86 93.98) (end 142.24 86.36) (width 0.75) (layer F.Cu) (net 2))
 (segment (start 149.86 107.95) (end 137.16 107.95) (width 0.75) (layer B.Cu) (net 2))
 (segment (start 149.86 95.25) (end 149.86 107.95) (width 0.75) (layer B.Cu) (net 2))
 (segment (start 142.24 86.36) (end 142.24 86.36) (width 0.75) (layer F.Cu) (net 2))
 (segment (start 124.46 60.96) (end 124.46 66.04) (width 0.5) (layer B.Cu) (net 8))
 (segment (start 95.25 92.71) (end 95.25 88.9) (width 0.5) (layer B.Cu) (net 8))
 (segment (start 98.425 88.9) (end 99.06 88.9) (width 0.5) (layer F.Cu) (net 8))
 (segment (start 95.25 88.9) (end 98.425 88.9) (width 0.5) (layer F.Cu) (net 8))
 (via (at 95.25 88.9) (size 0.6) (drill 0.5) (layers F.Cu B.Cu) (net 8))
 (segment (start 124.46 92.71) (end 113.03 92.71) (width 0.5) (layer B.Cu) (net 8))
 (segment (start 109.22 88.9) (end 99.06 88.9) (width 0.5) (layer F.Cu) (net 8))
 (segment (start 109.22 88.9) (end 113.03 92.71) (width 0.5) (layer F.Cu) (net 8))
 (via (at 113.03 92.71) (size 0.6) (drill 0.5) (layers F.Cu B.Cu) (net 8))
 (segment (start 99.06 88.9) (end 97.79 88.9) (width 0.5) (layer F.Cu) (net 8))
 (segment (start 95.25 92.71) (end 90.17 92.71) (width 0.5) (layer B.Cu) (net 8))
 (segment (start 86.36 71.12) (end 91.44 66.04) (width 0.5) (layer B.Cu) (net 8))
 (segment (start 86.36 88.9) (end 86.36 71.12) (width 0.5) (layer B.Cu) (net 8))
 (segment (start 90.17 92.71) (end 86.36 88.9) (width 0.5) (layer B.Cu) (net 8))
 (segment (start 124.46 66.04) (end 119.38 66.04) (width 0.5) (layer B.Cu) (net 8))
 (segment (start 103.505 57.785) (end 95.25 66.04) (width 0.5) (layer B.Cu) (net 8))
 (segment (start 95.25 66.04) (end 91.44 66.04) (width 0.5) (layer B.Cu) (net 8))
 (segment (start 111.125 57.785) (end 103.505 57.785) (width 0.5) (layer B.Cu) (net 8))
 (segment (start 119.38 66.04) (end 111.125 57.785) (width 0.5) (layer B.Cu) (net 8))
 (segment (start 127 60.96) (end 127 68.58) (width 0.5) (layer B.Cu) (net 9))
 (segment (start 127 68.58) (end 127 95.25) (width 0.5) (layer B.Cu) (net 9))
 (segment (start 127 95.25) (end 124.46 95.25) (width 0.5) (layer B.Cu) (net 9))
 (segment (start 127 68.58) (end 124.46 68.58) (width 0.5) (layer B.Cu) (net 9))
 (via (at 97.79 66.04) (size 0.6) (drill 0.5) (layers F.Cu B.Cu) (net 9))
 (segment (start 95.25 95.25) (end 97.79 95.25) (width 0.5) (layer B.Cu) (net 9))
 (segment (start 97.79 91.44) (end 97.79 95.25) (width 0.5) (layer B.Cu) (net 9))
 (segment (start 97.79 74.93) (end 97.79 91.44) (width 0.5) (layer B.Cu) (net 9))
 (via (at 97.79 74.93) (size 0.6) (drill 0.5) (layers F.Cu B.Cu) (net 9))
 (segment (start 97.79 74.93) (end 97.79 66.04) (width 0.5) (layer F.Cu) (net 9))
 (segment (start 124.46 68.58) (end 119.38 68.58) (width 0.5) (layer B.Cu) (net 9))
 (segment (start 119.38 68.58) (end 110.49 59.69) (width 0.5) (layer B.Cu) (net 9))
 (segment (start 110.49 59.69) (end 104.14 59.69) (width 0.5) (layer B.Cu) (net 9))
 (segment (start 104.14 59.69) (end 97.79 66.04) (width 0.5) (layer B.Cu) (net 9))
 (segment (start 97.79 66.04) (end 95.25 68.58) (width 0.5) (layer B.Cu) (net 9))
 (segment (start 128.905 71.12) (end 128.905 61.595) (width 0.5) (layer B.Cu) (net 10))
 (segment (start 128.905 61.595) (end 129.54 60.96) (width 0.5) (layer B.Cu) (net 10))
 (segment (start 128.905 71.12) (end 128.905 97.79) (width 0.5) (layer B.Cu) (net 10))
 (segment (start 128.905 97.79) (end 124.46 97.79) (width 0.5) (layer B.Cu) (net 10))
 (via (at 128.905 71.12) (size 0.6) (drill 0.5) (layers F.Cu B.Cu) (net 10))
 (segment (start 124.46 71.12) (end 125.73 71.12) (width 0.5) (layer B.Cu) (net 10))
 (via (at 125.73 71.12) (size 0.6) (drill 0.5) (layers F.Cu B.Cu) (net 10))
 (segment (start 125.73 71.12) (end 128.905 71.12) (width 0.5) (layer F.Cu) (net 10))
 (via (at 100.33 66.04) (size 0.6) (drill 0.5) (layers F.Cu B.Cu) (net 10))
 (segment (start 95.25 97.79) (end 100.33 97.79) (width 0.5) (layer B.Cu) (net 10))
 (segment (start 100.33 74.93) (end 100.33 97.79) (width 0.5) (layer B.Cu) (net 10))
 (via (at 100.33 74.93) (size 0.6) (drill 0.5) (layers F.Cu B.Cu) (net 10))
 (segment (start 100.33 74.93) (end 100.33 66.04) (width 0.5) (layer F.Cu) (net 10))
 (segment (start 124.46 71.12) (end 119.38 71.12) (width 0.5) (layer B.Cu) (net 10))
 (segment (start 104.775 61.595) (end 100.33 66.04) (width 0.5) (layer B.Cu) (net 10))
 (segment (start 100.33 66.04) (end 95.25 71.12) (width 0.5) (layer B.Cu) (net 10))
 (segment (start 109.855 61.595) (end 104.775 61.595) (width 0.5) (layer B.Cu) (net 10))
 (segment (start 119.38 71.12) (end 109.855 61.595) (width 0.5) (layer B.Cu) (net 10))
 (segment (start 130.81 73.66) (end 130.81 100.33) (width 0.5) (layer B.Cu) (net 11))
 (segment (start 130.81 100.33) (end 124.46 100.33) (width 0.5) (layer B.Cu) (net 11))
 (segment (start 130.81 73.66) (end 130.81 62.23) (width 0.5) (layer B.Cu) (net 11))
 (segment (start 130.81 62.23) (end 132.08 60.96) (width 0.5) (layer B.Cu) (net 11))
 (segment (start 124.46 73.66) (end 125.73 73.66) (width 0.5) (layer B.Cu) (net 11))
 (via (at 125.73 73.66) (size 0.6) (drill 0.5) (layers F.Cu B.Cu) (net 11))
 (via (at 130.81 73.66) (size 0.6) (drill 0.5) (layers F.Cu B.Cu) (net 11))
 (segment (start 130.81 73.66) (end 125.73 73.66) (width 0.5) (layer F.Cu) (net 11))
 (segment (start 102.87 66.04) (end 102.87 100.33) (width 0.5) (layer B.Cu) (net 11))
 (segment (start 102.87 100.33) (end 95.25 100.33) (width 0.5) (layer B.Cu) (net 11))
 (segment (start 124.46 73.66) (end 119.38 73.66) (width 0.5) (layer B.Cu) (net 11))
 (segment (start 105.41 63.5) (end 102.87 66.04) (width 0.5) (layer B.Cu) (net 11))
 (segment (start 102.87 66.04) (end 95.25 73.66) (width 0.5) (layer B.Cu) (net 11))
 (segment (start 109.22 63.5) (end 105.41 63.5) (width 0.5) (layer B.Cu) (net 11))
 (segment (start 119.38 73.66) (end 109.22 63.5) (width 0.5) (layer B.Cu) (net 11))
 (segment (start 95.25 83.82) (end 90.17 83.82) (width 0.5) (layer B.Cu) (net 28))
 (segment (start 90.17 81.28) (end 95.25 81.28) (width 0.5) (layer B.Cu) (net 27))
 (segment (start 95.25 110.49) (end 90.17 110.49) (width 0.5) (layer B.Cu) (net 21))
 (segment (start 90.17 107.95) (end 95.25 107.95) (width 0.5) (layer B.Cu) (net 20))
 (segment (start 119.38 83.82) (end 124.46 83.82) (width 0.5) (layer B.Cu) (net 29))
 (segment (start 124.46 81.28) (end 119.38 81.28) (width 0.5) (layer B.Cu) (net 30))
 (segment (start 124.46 110.49) (end 119.38 110.49) (width 0.5) (layer B.Cu) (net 14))
 (segment (start 119.38 107.95) (end 124.46 107.95) (width 0.5) (layer B.Cu) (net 13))
 (segment (start 113.03 78.74) (end 107.95 78.74) (width 0.75) (layer B.Cu) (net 22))
 (segment (start 107.95 76.2) (end 113.03 76.2) (width 0.75) (layer B.Cu) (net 23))
 (segment (start 113.03 73.66) (end 107.95 73.66) (width 0.75) (layer B.Cu) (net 24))
 (segment (start 107.95 71.12) (end 113.03 71.12) (width 0.75) (layer B.Cu) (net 25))
 (segment (start 95.25 76.2) (end 95.25 78.74) (width 0.5) (layer B.Cu) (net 26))
 (segment (start 113.03 105.41) (end 107.95 105.41) (width 0.75) (layer B.Cu) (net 15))
 (segment (start 107.95 102.87) (end 113.03 102.87) (width 0.75) (layer B.Cu) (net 16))
 (segment (start 107.95 100.33) (end 113.03 100.33) (width 0.75) (layer B.Cu) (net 17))
 (segment (start 113.03 97.79) (end 107.95 97.79) (width 0.75) (layer B.Cu) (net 18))
 (segment (start 95.25 102.87) (end 95.25 105.41) (width 0.5) (layer B.Cu) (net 19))
 (segment (start 142.24 78.74) (end 137.16 78.74) (width 0.75) (layer B.Cu) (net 31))
 (segment (start 142.24 76.2) (end 137.16 76.2) (width 0.75) (layer B.Cu) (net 32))
 (segment (start 137.16 73.66) (end 142.24 73.66) (width 0.75) (layer B.Cu) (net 33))
 (segment (start 142.24 71.12) (end 137.16 71.12) (width 0.75) (layer B.Cu) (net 34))
 (segment (start 124.46 76.2) (end 124.46 78.74) (width 0.5) (layer B.Cu) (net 35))
 (segment (start 137.16 105.41) (end 142.24 105.41) (width 0.75) (layer B.Cu) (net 3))
 (segment (start 142.24 102.87) (end 137.16 102.87) (width 0.75) (layer B.Cu) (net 4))
 (segment (start 142.24 100.33) (end 137.16 100.33) (width 0.75) (layer B.Cu) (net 5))
 (segment (start 137.16 97.79) (end 142.24 97.79) (width 0.75) (layer B.Cu) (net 6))
 (segment (start 124.46 105.41) (end 124.46 102.87) (width 0.5) (layer B.Cu) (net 12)))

